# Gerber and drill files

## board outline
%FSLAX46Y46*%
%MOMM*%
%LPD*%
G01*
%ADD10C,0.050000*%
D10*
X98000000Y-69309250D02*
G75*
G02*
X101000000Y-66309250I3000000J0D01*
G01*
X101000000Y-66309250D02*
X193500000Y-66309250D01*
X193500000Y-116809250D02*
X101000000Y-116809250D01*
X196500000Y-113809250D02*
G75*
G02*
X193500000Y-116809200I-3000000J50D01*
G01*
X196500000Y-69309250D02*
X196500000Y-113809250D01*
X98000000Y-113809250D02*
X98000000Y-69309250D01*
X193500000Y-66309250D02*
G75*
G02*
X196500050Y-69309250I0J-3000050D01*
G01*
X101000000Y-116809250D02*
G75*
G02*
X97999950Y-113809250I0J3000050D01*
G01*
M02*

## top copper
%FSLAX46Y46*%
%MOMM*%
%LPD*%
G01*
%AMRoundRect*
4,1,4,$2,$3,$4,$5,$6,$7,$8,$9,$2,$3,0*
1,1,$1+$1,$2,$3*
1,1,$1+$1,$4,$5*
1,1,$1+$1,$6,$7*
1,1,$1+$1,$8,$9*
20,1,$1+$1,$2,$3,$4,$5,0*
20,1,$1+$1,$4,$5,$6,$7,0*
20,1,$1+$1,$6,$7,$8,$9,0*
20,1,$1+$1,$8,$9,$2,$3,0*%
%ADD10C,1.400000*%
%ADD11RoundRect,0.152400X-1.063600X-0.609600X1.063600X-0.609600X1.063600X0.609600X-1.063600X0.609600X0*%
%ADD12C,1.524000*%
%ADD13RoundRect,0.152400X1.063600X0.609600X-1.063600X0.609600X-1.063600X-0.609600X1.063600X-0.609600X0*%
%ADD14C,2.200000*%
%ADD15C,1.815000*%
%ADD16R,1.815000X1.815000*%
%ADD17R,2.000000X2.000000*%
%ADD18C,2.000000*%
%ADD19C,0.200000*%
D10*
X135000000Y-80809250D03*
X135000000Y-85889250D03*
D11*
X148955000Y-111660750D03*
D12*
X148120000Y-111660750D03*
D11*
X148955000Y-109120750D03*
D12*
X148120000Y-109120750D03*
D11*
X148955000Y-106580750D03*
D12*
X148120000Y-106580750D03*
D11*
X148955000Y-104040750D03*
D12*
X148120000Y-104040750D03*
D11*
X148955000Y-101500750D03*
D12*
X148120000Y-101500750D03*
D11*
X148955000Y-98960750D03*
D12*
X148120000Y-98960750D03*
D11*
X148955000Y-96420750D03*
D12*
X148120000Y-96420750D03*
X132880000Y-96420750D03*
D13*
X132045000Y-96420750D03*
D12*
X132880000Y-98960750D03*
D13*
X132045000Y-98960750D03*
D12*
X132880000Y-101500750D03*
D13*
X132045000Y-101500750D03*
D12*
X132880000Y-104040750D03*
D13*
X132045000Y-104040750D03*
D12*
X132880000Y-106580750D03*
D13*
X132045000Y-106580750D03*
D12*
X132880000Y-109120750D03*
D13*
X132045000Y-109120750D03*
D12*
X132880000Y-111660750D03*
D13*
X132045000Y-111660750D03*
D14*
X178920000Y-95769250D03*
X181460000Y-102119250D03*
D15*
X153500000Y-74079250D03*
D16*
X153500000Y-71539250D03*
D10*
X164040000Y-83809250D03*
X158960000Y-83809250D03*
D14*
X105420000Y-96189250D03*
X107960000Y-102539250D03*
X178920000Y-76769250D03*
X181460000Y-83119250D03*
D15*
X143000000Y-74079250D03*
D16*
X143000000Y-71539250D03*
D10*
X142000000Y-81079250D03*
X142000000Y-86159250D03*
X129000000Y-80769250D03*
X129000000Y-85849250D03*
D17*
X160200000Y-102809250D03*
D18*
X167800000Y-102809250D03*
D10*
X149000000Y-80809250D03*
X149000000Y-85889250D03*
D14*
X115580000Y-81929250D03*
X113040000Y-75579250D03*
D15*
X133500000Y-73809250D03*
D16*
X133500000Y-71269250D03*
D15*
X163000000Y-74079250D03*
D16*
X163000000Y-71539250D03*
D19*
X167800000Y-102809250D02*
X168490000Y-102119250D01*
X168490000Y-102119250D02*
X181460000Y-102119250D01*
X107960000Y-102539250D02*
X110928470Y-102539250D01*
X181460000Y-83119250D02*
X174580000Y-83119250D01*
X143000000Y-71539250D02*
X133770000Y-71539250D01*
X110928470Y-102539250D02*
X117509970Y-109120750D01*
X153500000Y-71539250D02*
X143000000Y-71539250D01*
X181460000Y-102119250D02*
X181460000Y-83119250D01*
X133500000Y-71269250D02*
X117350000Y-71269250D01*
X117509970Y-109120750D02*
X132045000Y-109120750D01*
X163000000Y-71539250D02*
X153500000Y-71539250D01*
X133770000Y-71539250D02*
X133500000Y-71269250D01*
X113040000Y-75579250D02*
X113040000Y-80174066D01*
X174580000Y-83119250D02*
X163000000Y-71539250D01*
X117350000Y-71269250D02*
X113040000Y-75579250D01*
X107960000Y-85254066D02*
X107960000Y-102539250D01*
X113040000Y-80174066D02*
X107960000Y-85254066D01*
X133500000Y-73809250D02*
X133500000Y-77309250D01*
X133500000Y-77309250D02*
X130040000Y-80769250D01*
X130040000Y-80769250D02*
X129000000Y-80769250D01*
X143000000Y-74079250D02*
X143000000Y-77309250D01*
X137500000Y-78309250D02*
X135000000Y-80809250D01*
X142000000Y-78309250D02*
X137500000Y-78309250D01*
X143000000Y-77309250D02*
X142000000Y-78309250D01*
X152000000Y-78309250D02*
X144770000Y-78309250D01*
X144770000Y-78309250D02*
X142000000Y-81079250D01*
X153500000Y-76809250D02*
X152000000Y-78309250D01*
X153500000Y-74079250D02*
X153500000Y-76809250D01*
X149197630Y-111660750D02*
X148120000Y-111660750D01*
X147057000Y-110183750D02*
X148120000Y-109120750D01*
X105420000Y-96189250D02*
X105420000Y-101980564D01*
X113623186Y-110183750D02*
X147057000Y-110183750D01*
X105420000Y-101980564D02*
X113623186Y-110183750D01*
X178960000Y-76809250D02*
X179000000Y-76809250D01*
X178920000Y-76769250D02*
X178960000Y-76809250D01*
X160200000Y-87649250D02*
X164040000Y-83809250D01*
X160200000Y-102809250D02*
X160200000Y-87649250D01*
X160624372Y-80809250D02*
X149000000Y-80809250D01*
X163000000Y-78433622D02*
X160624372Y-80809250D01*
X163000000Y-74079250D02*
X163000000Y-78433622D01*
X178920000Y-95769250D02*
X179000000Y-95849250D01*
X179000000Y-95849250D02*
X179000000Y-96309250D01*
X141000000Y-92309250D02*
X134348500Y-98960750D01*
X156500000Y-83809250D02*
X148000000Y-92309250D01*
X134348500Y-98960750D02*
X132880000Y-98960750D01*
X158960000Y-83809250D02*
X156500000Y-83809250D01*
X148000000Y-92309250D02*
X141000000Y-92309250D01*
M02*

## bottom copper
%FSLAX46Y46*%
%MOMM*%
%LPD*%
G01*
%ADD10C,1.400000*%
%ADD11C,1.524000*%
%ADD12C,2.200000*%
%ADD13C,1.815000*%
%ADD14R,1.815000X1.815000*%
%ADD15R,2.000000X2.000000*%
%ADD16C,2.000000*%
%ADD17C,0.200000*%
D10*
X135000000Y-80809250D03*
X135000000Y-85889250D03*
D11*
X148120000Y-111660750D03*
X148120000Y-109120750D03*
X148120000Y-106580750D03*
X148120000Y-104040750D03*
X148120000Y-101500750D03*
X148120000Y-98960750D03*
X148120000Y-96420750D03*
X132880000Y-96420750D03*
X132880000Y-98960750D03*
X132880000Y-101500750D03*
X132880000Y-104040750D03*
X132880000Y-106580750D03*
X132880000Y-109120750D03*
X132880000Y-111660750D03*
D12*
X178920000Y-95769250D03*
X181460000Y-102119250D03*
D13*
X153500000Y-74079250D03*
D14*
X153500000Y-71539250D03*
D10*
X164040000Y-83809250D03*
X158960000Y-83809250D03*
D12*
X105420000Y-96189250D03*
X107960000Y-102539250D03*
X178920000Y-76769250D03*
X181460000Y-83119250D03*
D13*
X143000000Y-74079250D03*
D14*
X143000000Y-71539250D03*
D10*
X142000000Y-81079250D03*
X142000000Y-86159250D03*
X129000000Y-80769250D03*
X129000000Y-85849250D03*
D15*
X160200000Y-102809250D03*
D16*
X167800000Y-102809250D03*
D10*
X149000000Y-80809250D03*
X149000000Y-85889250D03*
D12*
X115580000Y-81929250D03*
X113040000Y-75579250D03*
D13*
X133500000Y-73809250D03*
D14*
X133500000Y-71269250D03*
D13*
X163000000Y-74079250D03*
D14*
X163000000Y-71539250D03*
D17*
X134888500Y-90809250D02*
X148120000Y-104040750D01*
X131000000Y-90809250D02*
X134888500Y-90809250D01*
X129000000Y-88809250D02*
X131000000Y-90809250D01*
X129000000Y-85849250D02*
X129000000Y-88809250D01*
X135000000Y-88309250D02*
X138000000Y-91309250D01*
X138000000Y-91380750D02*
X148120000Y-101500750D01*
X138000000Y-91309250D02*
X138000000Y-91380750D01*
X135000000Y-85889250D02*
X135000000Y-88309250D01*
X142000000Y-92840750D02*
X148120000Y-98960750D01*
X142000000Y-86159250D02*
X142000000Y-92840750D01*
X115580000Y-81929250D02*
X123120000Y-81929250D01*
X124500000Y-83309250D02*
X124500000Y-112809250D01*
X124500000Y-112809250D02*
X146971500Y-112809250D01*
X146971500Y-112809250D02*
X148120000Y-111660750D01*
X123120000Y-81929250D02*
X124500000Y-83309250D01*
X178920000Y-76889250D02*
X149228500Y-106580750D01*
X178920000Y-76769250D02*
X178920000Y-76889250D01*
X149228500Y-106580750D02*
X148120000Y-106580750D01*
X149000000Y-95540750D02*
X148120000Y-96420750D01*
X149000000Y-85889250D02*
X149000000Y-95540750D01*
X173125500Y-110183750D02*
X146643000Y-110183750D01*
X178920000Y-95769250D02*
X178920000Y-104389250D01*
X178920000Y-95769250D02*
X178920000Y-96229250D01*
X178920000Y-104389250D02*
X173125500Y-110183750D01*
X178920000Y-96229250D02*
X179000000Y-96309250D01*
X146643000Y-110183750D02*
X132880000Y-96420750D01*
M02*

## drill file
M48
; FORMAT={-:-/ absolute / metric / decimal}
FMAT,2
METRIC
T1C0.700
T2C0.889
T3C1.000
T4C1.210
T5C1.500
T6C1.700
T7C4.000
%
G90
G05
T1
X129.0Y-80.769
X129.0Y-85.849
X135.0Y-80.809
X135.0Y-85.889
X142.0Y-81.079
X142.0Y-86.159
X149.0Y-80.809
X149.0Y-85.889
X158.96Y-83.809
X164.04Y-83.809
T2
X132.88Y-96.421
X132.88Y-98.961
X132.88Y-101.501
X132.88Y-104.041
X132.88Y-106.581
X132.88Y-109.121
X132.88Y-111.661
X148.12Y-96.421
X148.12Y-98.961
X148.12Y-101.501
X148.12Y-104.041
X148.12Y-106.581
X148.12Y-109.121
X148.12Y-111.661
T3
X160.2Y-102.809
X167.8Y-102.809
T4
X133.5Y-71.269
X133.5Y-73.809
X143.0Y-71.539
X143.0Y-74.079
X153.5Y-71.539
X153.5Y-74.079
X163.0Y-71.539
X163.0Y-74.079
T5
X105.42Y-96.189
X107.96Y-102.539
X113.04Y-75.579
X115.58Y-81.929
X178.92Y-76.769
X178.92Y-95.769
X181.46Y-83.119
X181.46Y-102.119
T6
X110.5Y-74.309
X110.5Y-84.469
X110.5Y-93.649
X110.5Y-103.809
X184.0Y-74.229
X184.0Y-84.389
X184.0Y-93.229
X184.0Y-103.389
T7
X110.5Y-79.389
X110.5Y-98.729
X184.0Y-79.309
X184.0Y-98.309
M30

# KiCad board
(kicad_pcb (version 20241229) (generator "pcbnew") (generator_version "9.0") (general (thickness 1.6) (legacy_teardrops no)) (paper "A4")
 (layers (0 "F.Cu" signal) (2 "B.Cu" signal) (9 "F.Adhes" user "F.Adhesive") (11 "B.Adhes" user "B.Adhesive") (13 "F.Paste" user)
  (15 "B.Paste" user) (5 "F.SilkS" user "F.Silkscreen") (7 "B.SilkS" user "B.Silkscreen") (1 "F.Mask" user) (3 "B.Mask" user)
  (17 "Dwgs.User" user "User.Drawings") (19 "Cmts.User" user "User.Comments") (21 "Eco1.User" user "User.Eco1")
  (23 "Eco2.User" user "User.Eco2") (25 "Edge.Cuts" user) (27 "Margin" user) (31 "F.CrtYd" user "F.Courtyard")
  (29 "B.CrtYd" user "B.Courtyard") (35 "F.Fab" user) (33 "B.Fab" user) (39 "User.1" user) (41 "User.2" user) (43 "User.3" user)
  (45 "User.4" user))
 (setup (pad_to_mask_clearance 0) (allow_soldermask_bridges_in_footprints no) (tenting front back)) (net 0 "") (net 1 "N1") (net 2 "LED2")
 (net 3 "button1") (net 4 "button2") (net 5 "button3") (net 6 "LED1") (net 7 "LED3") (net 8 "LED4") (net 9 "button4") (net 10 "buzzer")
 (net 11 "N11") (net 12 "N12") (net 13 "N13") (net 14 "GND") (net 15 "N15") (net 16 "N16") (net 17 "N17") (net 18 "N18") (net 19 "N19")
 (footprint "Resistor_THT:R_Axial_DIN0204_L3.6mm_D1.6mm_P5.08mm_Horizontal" (layer "F.Cu") (at 135 80.80925 -90)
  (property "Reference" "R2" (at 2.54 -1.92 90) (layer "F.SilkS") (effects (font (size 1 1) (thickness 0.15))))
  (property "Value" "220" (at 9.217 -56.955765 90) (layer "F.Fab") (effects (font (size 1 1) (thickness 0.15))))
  (pad "1" thru_hole circle (at 0 0 270) (size 1.4 1.4) (drill 0.7) (layers "*.Cu" "*.Mask") (remove_unused_layers no) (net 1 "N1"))
  (pad "2" thru_hole circle (at 5.08 0 270) (size 1.4 1.4) (drill 0.7) (layers "*.Cu" "*.Mask") (remove_unused_layers no) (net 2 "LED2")))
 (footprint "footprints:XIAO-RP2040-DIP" (layer "F.Cu") (at 140.5 104.04075 -90)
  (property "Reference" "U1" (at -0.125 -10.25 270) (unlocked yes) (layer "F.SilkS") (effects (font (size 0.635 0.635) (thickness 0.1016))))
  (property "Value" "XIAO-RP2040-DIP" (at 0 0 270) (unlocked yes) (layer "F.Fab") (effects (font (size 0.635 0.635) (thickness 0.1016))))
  (pad "1" smd roundrect (at 7.62 -8.455) (size 2.432 1.524) (layers "F.Cu" "F.Mask") (roundrect_rratio 0.1) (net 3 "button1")
   (thermal_bridge_angle 45))
  (pad "1" thru_hole circle (at 7.62 -7.62) (size 1.524 1.524) (drill 0.889) (layers "*.Cu" "*.Mask") (remove_unused_layers no)
   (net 3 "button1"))
  (pad "2" smd roundrect (at 5.08 -8.455) (size 2.432 1.524) (layers "F.Cu" "F.Mask") (roundrect_rratio 0.1) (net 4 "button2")
   (thermal_bridge_angle 45))
  (pad "2" thru_hole circle (at 5.08 -7.62) (size 1.524 1.524) (drill 0.889) (layers "*.Cu" "*.Mask") (remove_unused_layers no)
   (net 4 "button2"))
  (pad "3" smd roundrect (at 2.54 -8.455) (size 2.432 1.524) (layers "F.Cu" "F.Mask") (roundrect_rratio 0.1) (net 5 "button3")
   (thermal_bridge_angle 45))
  (pad "3" thru_hole circle (at 2.54 -7.62) (size 1.524 1.524) (drill 0.889) (layers "*.Cu" "*.Mask") (remove_unused_layers no)
   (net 5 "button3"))
  (pad "4" smd roundrect (at 0 -8.455) (size 2.432 1.524) (layers "F.Cu" "F.Mask") (roundrect_rratio 0.1) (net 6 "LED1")
   (thermal_bridge_angle 45))
  (pad "4" thru_hole circle (at 0 -7.62) (size 1.524 1.524) (drill 0.889) (layers "*.Cu" "*.Mask") (remove_unused_layers no) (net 6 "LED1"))
  (pad "5" smd roundrect (at -2.54 -8.455) (size 2.432 1.524) (layers "F.Cu" "F.Mask") (roundrect_rratio 0.1) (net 2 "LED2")
   (thermal_bridge_angle 45))
  (pad "5" thru_hole circle (at -2.54 -7.62) (size 1.524 1.524) (drill 0.889) (layers "*.Cu" "*.Mask") (remove_unused_layers no)
   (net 2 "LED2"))
  (pad "6" smd roundrect (at -5.08 -8.455) (size 2.432 1.524) (layers "F.Cu" "F.Mask") (roundrect_rratio 0.1) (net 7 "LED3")
   (thermal_bridge_angle 45))
  (pad "6" thru_hole circle (at -5.08 -7.62) (size 1.524 1.524) (drill 0.889) (layers "*.Cu" "*.Mask") (remove_unused_layers no)
   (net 7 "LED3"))
  (pad "7" smd roundrect (at -7.62 -8.455) (size 2.432 1.524) (layers "F.Cu" "F.Mask") (roundrect_rratio 0.1) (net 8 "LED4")
   (thermal_bridge_angle 45))
  (pad "7" thru_hole circle (at -7.62 -7.62) (size 1.524 1.524) (drill 0.889) (layers "*.Cu" "*.Mask") (remove_unused_layers no)
   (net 8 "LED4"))
  (pad "8" thru_hole circle (at -7.62 7.62 180) (size 1.524 1.524) (drill 0.889) (layers "*.Cu" "*.Mask") (remove_unused_layers no)
   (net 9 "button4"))
  (pad "8" smd roundrect (at -7.62 8.455 180) (size 2.432 1.524) (layers "F.Cu" "F.Mask") (roundrect_rratio 0.1) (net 9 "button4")
   (thermal_bridge_angle 45))
  (pad "9" thru_hole circle (at -5.08 7.62 180) (size 1.524 1.524) (drill 0.889) (layers "*.Cu" "*.Mask") (remove_unused_layers no)
   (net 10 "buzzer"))
  (pad "9" smd roundrect (at -5.08 8.455 180) (size 2.432 1.524) (layers "F.Cu" "F.Mask") (roundrect_rratio 0.1) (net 10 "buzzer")
   (thermal_bridge_angle 45))
  (pad "10" thru_hole circle (at -2.54 7.62 180) (size 1.524 1.524) (drill 0.889) (layers "*.Cu" "*.Mask") (remove_unused_layers no)
   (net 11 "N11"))
  (pad "10" smd roundrect (at -2.54 8.455 180) (size 2.432 1.524) (layers "F.Cu" "F.Mask") (roundrect_rratio 0.1) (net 11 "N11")
   (thermal_bridge_angle 45))
  (pad "11" thru_hole circle (at 0 7.62 180) (size 1.524 1.524) (drill 0.889) (layers "*.Cu" "*.Mask") (remove_unused_layers no)
   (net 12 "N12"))
  (pad "11" smd roundrect (at 0 8.455 180) (size 2.432 1.524) (layers "F.Cu" "F.Mask") (roundrect_rratio 0.1) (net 12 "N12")
   (thermal_bridge_angle 45))
  (pad "12" thru_hole circle (at 2.54 7.62 180) (size 1.524 1.524) (drill 0.889) (layers "*.Cu" "*.Mask") (remove_unused_layers no)
   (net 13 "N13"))
  (pad "12" smd roundrect (at 2.54 8.455 180) (size 2.432 1.524) (layers "F.Cu" "F.Mask") (roundrect_rratio 0.1) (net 13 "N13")
   (thermal_bridge_angle 45))
  (pad "13" thru_hole circle (at 5.08 7.62 180) (size 1.524 1.524) (drill 0.889) (layers "*.Cu" "*.Mask") (remove_unused_layers no)
   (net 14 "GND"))
  (pad "13" smd roundrect (at 5.08 8.455 180) (size 2.432 1.524) (layers "F.Cu" "F.Mask") (roundrect_rratio 0.1) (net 14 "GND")
   (thermal_bridge_angle 45))
  (pad "14" thru_hole circle (at 7.62 7.62 180) (size 1.524 1.524) (drill 0.889) (layers "*.Cu" "*.Mask") (remove_unused_layers no)
   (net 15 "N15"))
  (pad "14" smd roundrect (at 7.62 8.455 180) (size 2.432 1.524) (layers "F.Cu" "F.Mask") (roundrect_rratio 0.1) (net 15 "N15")
   (thermal_bridge_angle 45)))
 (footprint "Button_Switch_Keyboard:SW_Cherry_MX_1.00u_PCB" (layer "F.Cu") (at 178.92 95.76925 90)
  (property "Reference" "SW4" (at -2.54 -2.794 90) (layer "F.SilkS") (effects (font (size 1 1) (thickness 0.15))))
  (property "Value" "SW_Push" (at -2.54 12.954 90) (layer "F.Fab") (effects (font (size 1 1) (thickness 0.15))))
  (pad "" np_thru_hole circle (at -7.62 5.08 90) (size 1.7 1.7) (drill 1.7) (layers "*.Cu" "*.Mask"))
  (pad "" np_thru_hole circle (at -2.54 5.08 90) (size 4 4) (drill 4) (layers "*.Cu" "*.Mask"))
  (pad "" np_thru_hole circle (at 2.54 5.08 90) (size 1.7 1.7) (drill 1.7) (layers "*.Cu" "*.Mask"))
  (pad "1" thru_hole circle (at 0 0 90) (size 2.2 2.2) (drill 1.5) (layers "*.Cu" "*.Mask") (remove_unused_layers no) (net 9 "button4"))
  (pad "2" thru_hole circle (at -6.35 2.54 90) (size 2.2 2.2) (drill 1.5) (layers "*.Cu" "*.Mask") (remove_unused_layers no) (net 14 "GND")))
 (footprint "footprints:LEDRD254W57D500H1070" (layer "F.Cu") (at 153.5 72.80925 -90)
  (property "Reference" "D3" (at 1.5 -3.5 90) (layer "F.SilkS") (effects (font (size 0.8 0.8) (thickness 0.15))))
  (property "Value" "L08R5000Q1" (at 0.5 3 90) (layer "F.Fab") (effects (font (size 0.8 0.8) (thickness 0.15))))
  (pad "A" thru_hole circle (at 1.27 0 270) (size 1.815 1.815) (drill 1.21) (layers "*.Cu" "*.Mask") (remove_unused_layers no)
   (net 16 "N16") (solder_mask_margin 0.102))
  (pad "C" thru_hole rect (at -1.27 0 270) (size 1.815 1.815) (drill 1.21) (layers "*.Cu" "*.Mask") (remove_unused_layers no) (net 14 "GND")
   (solder_mask_margin 0.102)))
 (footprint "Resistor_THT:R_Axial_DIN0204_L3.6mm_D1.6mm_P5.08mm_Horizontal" (layer "F.Cu") (at 164.04 83.80925 180)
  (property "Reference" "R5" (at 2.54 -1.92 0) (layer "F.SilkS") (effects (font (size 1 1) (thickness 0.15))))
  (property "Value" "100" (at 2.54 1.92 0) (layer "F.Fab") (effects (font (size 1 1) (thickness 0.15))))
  (pad "1" thru_hole circle (at 0 0 180) (size 1.4 1.4) (drill 0.7) (layers "*.Cu" "*.Mask") (remove_unused_layers no) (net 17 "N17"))
  (pad "2" thru_hole circle (at 5.08 0 180) (size 1.4 1.4) (drill 0.7) (layers "*.Cu" "*.Mask") (remove_unused_layers no) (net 10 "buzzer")))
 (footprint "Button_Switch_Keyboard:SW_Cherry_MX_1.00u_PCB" (layer "F.Cu") (at 105.42 96.18925 90)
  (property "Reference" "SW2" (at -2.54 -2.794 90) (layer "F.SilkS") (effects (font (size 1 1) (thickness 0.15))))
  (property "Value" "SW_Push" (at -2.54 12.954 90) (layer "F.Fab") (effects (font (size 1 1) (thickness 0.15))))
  (pad "" np_thru_hole circle (at -7.62 5.08 90) (size 1.7 1.7) (drill 1.7) (layers "*.Cu" "*.Mask"))
  (pad "" np_thru_hole circle (at -2.54 5.08 90) (size 4 4) (drill 4) (layers "*.Cu" "*.Mask"))
  (pad "" np_thru_hole circle (at 2.54 5.08 90) (size 1.7 1.7) (drill 1.7) (layers "*.Cu" "*.Mask"))
  (pad "1" thru_hole circle (at 0 0 90) (size 2.2 2.2) (drill 1.5) (layers "*.Cu" "*.Mask") (remove_unused_layers no) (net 4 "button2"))
  (pad "2" thru_hole circle (at -6.35 2.54 90) (size 2.2 2.2) (drill 1.5) (layers "*.Cu" "*.Mask") (remove_unused_layers no) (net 14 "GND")))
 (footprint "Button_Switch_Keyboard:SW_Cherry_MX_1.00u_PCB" (layer "F.Cu") (at 178.92 76.76925 90)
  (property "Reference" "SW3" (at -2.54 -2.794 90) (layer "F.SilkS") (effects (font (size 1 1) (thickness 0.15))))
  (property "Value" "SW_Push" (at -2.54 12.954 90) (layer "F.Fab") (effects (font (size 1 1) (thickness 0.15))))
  (pad "" np_thru_hole circle (at -7.62 5.08 90) (size 1.7 1.7) (drill 1.7) (layers "*.Cu" "*.Mask"))
  (pad "" np_thru_hole circle (at -2.54 5.08 90) (size 4 4) (drill 4) (layers "*.Cu" "*.Mask"))
  (pad "" np_thru_hole circle (at 2.54 5.08 90) (size 1.7 1.7) (drill 1.7) (layers "*.Cu" "*.Mask"))
  (pad "1" thru_hole circle (at 0 0 90) (size 2.2 2.2) (drill 1.5) (layers "*.Cu" "*.Mask") (remove_unused_layers no) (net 5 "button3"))
  (pad "2" thru_hole circle (at -6.35 2.54 90) (size 2.2 2.2) (drill 1.5) (layers "*.Cu" "*.Mask") (remove_unused_layers no) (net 14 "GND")))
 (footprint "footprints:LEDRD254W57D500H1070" (layer "F.Cu") (at 143 72.80925 -90)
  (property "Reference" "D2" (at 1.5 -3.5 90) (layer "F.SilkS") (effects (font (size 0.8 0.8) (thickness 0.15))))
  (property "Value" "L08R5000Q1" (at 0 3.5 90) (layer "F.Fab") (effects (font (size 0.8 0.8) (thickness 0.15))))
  (pad "A" thru_hole circle (at 1.27 0 270) (size 1.815 1.815) (drill 1.21) (layers "*.Cu" "*.Mask") (remove_unused_layers no) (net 1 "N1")
   (solder_mask_margin 0.102))
  (pad "C" thru_hole rect (at -1.27 0 270) (size 1.815 1.815) (drill 1.21) (layers "*.Cu" "*.Mask") (remove_unused_layers no) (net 14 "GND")
   (solder_mask_margin 0.102)))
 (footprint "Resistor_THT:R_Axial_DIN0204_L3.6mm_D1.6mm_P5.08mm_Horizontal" (layer "F.Cu") (at 142 81.07925 -90)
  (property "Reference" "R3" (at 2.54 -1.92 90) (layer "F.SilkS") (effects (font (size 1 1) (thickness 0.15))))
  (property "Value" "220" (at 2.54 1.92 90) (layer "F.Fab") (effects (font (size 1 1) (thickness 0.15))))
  (pad "1" thru_hole circle (at 0 0 270) (size 1.4 1.4) (drill 0.7) (layers "*.Cu" "*.Mask") (remove_unused_layers no) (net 16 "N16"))
  (pad "2" thru_hole circle (at 5.08 0 270) (size 1.4 1.4) (drill 0.7) (layers "*.Cu" "*.Mask") (remove_unused_layers no) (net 7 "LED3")))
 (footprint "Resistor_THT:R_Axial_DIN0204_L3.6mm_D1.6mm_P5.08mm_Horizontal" (layer "F.Cu") (at 129 80.76925 -90)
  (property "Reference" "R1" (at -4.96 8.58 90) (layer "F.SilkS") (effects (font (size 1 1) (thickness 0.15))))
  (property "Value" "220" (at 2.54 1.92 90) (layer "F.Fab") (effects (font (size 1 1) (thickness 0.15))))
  (pad "1" thru_hole circle (at 0 0 270) (size 1.4 1.4) (drill 0.7) (layers "*.Cu" "*.Mask") (remove_unused_layers no) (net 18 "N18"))
  (pad "2" thru_hole circle (at 5.08 0 270) (size 1.4 1.4) (drill 0.7) (layers "*.Cu" "*.Mask") (remove_unused_layers no) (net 6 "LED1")))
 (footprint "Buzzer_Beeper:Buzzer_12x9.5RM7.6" (layer "F.Cu") (at 160.2 102.80925)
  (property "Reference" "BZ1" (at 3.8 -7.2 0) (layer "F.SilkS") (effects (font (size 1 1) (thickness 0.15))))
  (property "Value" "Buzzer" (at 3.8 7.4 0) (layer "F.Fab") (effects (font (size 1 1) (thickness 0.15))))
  (pad "1" thru_hole rect (at 0 0) (size 2 2) (drill 1) (layers "*.Cu" "*.Mask") (remove_unused_layers no) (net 17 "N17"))
  (pad "2" thru_hole circle (at 7.6 0) (size 2 2) (drill 1) (layers "*.Cu" "*.Mask") (remove_unused_layers no) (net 14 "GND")))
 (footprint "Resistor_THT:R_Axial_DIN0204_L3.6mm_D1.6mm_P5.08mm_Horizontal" (layer "F.Cu") (at 149 80.80925 -90)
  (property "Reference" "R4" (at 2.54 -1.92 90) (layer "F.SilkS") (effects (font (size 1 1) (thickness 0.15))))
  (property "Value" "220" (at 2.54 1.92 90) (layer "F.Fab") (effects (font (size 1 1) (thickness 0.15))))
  (pad "1" thru_hole circle (at 0 0 270) (size 1.4 1.4) (drill 0.7) (layers "*.Cu" "*.Mask") (remove_unused_layers no) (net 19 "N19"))
  (pad "2" thru_hole circle (at 5.08 0 270) (size 1.4 1.4) (drill 0.7) (layers "*.Cu" "*.Mask") (remove_unused_layers no) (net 8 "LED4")))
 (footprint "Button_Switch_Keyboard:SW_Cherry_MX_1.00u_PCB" (layer "F.Cu") (at 115.58 81.92925 -90)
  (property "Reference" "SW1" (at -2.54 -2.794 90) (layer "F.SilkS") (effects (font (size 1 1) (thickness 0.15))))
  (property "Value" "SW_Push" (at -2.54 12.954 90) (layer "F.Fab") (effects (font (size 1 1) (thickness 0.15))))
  (pad "" np_thru_hole circle (at -7.62 5.08 270) (size 1.7 1.7) (drill 1.7) (layers "*.Cu" "*.Mask"))
  (pad "" np_thru_hole circle (at -2.54 5.08 270) (size 4 4) (drill 4) (layers "*.Cu" "*.Mask"))
  (pad "" np_thru_hole circle (at 2.54 5.08 270) (size 1.7 1.7) (drill 1.7) (layers "*.Cu" "*.Mask"))
  (pad "1" thru_hole circle (at 0 0 270) (size 2.2 2.2) (drill 1.5) (layers "*.Cu" "*.Mask") (remove_unused_layers no) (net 3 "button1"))
  (pad "2" thru_hole circle (at -6.35 2.54 270) (size 2.2 2.2) (drill 1.5) (layers "*.Cu" "*.Mask") (remove_unused_layers no) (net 14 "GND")))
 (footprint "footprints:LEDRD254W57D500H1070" (layer "F.Cu") (at 133.5 72.53925 -90)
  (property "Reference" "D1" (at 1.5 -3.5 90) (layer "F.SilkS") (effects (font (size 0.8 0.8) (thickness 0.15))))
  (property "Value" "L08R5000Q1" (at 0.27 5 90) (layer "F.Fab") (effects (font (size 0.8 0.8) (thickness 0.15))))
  (pad "A" thru_hole circle (at 1.27 0 270) (size 1.815 1.815) (drill 1.21) (layers "*.Cu" "*.Mask") (remove_unused_layers no)
   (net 18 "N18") (solder_mask_margin 0.102))
  (pad "C" thru_hole rect (at -1.27 0 270) (size 1.815 1.815) (drill 1.21) (layers "*.Cu" "*.Mask") (remove_unused_layers no) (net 14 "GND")
   (solder_mask_margin 0.102)))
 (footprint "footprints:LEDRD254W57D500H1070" (layer "F.Cu") (at 163 72.80925 -90)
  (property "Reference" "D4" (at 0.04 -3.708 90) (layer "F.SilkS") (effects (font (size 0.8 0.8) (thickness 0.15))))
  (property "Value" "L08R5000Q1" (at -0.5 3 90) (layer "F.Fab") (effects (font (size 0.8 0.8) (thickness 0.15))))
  (pad "A" thru_hole circle (at 1.27 0 270) (size 1.815 1.815) (drill 1.21) (layers "*.Cu" "*.Mask") (remove_unused_layers no)
   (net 19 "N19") (solder_mask_margin 0.102))
  (pad "C" thru_hole rect (at -1.27 0 270) (size 1.815 1.815) (drill 1.21) (layers "*.Cu" "*.Mask") (remove_unused_layers no) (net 14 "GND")
   (solder_mask_margin 0.102)))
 (gr_arc (start 98 69.30925) (mid 98.87868 67.18793) (end 101 66.30925) (stroke (width 0.05) (type default)) (layer "Edge.Cuts"))
 (gr_line (start 101 66.30925) (end 193.5 66.30925) (stroke (width 0.05) (type default)) (layer "Edge.Cuts"))
 (gr_line (start 193.5 116.80925) (end 101 116.80925) (stroke (width 0.05) (type default)) (layer "Edge.Cuts"))
 (gr_arc (start 196.5 113.80925) (mid 195.62132 115.93057) (end 193.5 116.80925) (stroke (width 0.05) (type default)) (layer "Edge.Cuts"))
 (gr_line (start 196.5 69.30925) (end 196.5 113.80925) (stroke (width 0.05) (type default)) (layer "Edge.Cuts"))
 (gr_line (start 98 113.80925) (end 98 69.30925) (stroke (width 0.05) (type default)) (layer "Edge.Cuts"))
 (gr_arc (start 193.5 66.30925) (mid 195.62132 67.18793) (end 196.5 69.30925) (stroke (width 0.05) (type default)) (layer "Edge.Cuts"))
 (gr_arc (start 101 116.80925) (mid 98.87868 115.93057) (end 98 113.80925) (stroke (width 0.05) (type default)) (layer "Edge.Cuts"))
 (segment (start 167.8 102.80925) (end 168.49 102.11925) (width 0.2) (layer "F.Cu") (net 14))
 (segment (start 168.49 102.11925) (end 181.46 102.11925) (width 0.2) (layer "F.Cu") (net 14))
 (segment (start 107.96 102.53925) (end 110.92847 102.53925) (width 0.2) (layer "F.Cu") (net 14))
 (segment (start 181.46 83.11925) (end 174.58 83.11925) (width 0.2) (layer "F.Cu") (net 14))
 (segment (start 143 71.53925) (end 133.77 71.53925) (width 0.2) (layer "F.Cu") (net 14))
 (segment (start 110.92847 102.53925) (end 117.50997 109.12075) (width 0.2) (layer "F.Cu") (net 14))
 (segment (start 153.5 71.53925) (end 143 71.53925) (width 0.2) (layer "F.Cu") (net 14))
 (segment (start 181.46 102.11925) (end 181.46 83.11925) (width 0.2) (layer "F.Cu") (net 14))
 (segment (start 133.5 71.26925) (end 117.35 71.26925) (width 0.2) (layer "F.Cu") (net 14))
 (segment (start 117.50997 109.12075) (end 132.045 109.12075) (width 0.2) (layer "F.Cu") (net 14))
 (segment (start 163 71.53925) (end 153.5 71.53925) (width 0.2) (layer "F.Cu") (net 14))
 (segment (start 133.77 71.53925) (end 133.5 71.26925) (width 0.2) (layer "F.Cu") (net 14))
 (segment (start 113.04 75.57925) (end 113.04 80.174066) (width 0.2) (layer "F.Cu") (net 14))
 (segment (start 174.58 83.11925) (end 163 71.53925) (width 0.2) (layer "F.Cu") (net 14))
 (segment (start 117.35 71.26925) (end 113.04 75.57925) (width 0.2) (layer "F.Cu") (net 14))
 (segment (start 107.96 85.254066) (end 107.96 102.53925) (width 0.2) (layer "F.Cu") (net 14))
 (segment (start 113.04 80.174066) (end 107.96 85.254066) (width 0.2) (layer "F.Cu") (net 14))
 (segment (start 133.5 73.80925) (end 133.5 77.30925) (width 0.2) (layer "F.Cu") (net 18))
 (segment (start 133.5 77.30925) (end 130.04 80.76925) (width 0.2) (layer "F.Cu") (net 18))
 (segment (start 130.04 80.76925) (end 129 80.76925) (width 0.2) (layer "F.Cu") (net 18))
 (segment (start 143 74.07925) (end 143 77.30925) (width 0.2) (layer "F.Cu") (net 1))
 (segment (start 137.5 78.30925) (end 135 80.80925) (width 0.2) (layer "F.Cu") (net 1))
 (segment (start 142 78.30925) (end 137.5 78.30925) (width 0.2) (layer "F.Cu") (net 1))
 (segment (start 143 77.30925) (end 142 78.30925) (width 0.2) (layer "F.Cu") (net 1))
 (segment (start 152 78.30925) (end 144.77 78.30925) (width 0.2) (layer "F.Cu") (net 16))
 (segment (start 144.77 78.30925) (end 142 81.07925) (width 0.2) (layer "F.Cu") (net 16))
 (segment (start 153.5 76.80925) (end 152 78.30925) (width 0.2) (layer "F.Cu") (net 16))
 (segment (start 153.5 74.07925) (end 153.5 76.80925) (width 0.2) (layer "F.Cu") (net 16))
 (segment (start 134.8885 90.80925) (end 148.12 104.04075) (width 0.2) (layer "B.Cu") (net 6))
 (segment (start 131 90.80925) (end 134.8885 90.80925) (width 0.2) (layer "B.Cu") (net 6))
 (segment (start 129 88.80925) (end 131 90.80925) (width 0.2) (layer "B.Cu") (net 6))
 (segment (start 129 85.84925) (end 129 88.80925) (width 0.2) (layer "B.Cu") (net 6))
 (segment (start 135 88.30925) (end 138 91.30925) (width 0.2) (layer "B.Cu") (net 2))
 (segment (start 138 91.38075) (end 148.12 101.50075) (width 0.2) (layer "B.Cu") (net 2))
 (segment (start 138 91.30925) (end 138 91.38075) (width 0.2) (layer "B.Cu") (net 2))
 (segment (start 135 85.88925) (end 135 88.30925) (width 0.2) (layer "B.Cu") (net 2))
 (segment (start 142 92.84075) (end 148.12 98.96075) (width 0.2) (layer "B.Cu") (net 7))
 (segment (start 142 86.15925) (end 142 92.84075) (width 0.2) (layer "B.Cu") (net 7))
 (segment (start 149.19763 111.66075) (end 148.12 111.66075) (width 0.2) (layer "F.Cu") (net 3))
 (segment (start 115.58 81.92925) (end 123.12 81.92925) (width 0.2) (layer "B.Cu") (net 3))
 (segment (start 124.5 83.30925) (end 124.5 112.80925) (width 0.2) (layer "B.Cu") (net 3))
 (segment (start 124.5 112.80925) (end 146.9715 112.80925) (width 0.2) (layer "B.Cu") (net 3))
 (segment (start 146.9715 112.80925) (end 148.12 111.66075) (width 0.2) (layer "B.Cu") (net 3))
 (segment (start 123.12 81.92925) (end 124.5 83.30925) (width 0.2) (layer "B.Cu") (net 3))
 (segment (start 147.057 110.18375) (end 148.12 109.12075) (width 0.2) (layer "F.Cu") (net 4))
 (segment (start 105.42 96.18925) (end 105.42 101.980564) (width 0.2) (layer "F.Cu") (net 4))
 (segment (start 113.623186 110.18375) (end 147.057 110.18375) (width 0.2) (layer "F.Cu") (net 4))
 (segment (start 105.42 101.980564) (end 113.623186 110.18375) (width 0.2) (layer "F.Cu") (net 4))
 (segment (start 178.96 76.80925) (end 179 76.80925) (width 0.2) (layer "F.Cu") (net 5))
 (segment (start 178.92 76.76925) (end 178.96 76.80925) (width 0.2) (layer "F.Cu") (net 5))
 (segment (start 178.92 76.88925) (end 149.2285 106.58075) (width 0.2) (layer "B.Cu") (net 5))
 (segment (start 178.92 76.76925) (end 178.92 76.88925) (width 0.2) (layer "B.Cu") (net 5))
 (segment (start 149.2285 106.58075) (end 148.12 106.58075) (width 0.2) (layer "B.Cu") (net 5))
 (segment (start 160.2 87.64925) (end 164.04 83.80925) (width 0.2) (layer "F.Cu") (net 17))
 (segment (start 160.2 102.80925) (end 160.2 87.64925) (width 0.2) (layer "F.Cu") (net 17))
 (segment (start 160.624372 80.80925) (end 149 80.80925) (width 0.2) (layer "F.Cu") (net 19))
 (segment (start 163 78.433622) (end 160.624372 80.80925) (width 0.2) (layer "F.Cu") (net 19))
 (segment (start 163 74.07925) (end 163 78.433622) (width 0.2) (layer "F.Cu") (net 19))
 (segment (start 149 95.54075) (end 148.12 96.42075) (width 0.2) (layer "B.Cu") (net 8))
 (segment (start 149 85.88925) (end 149 95.54075) (width 0.2) (layer "B.Cu") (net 8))
 (segment (start 178.92 95.76925) (end 179 95.84925) (width 0.2) (layer "F.Cu") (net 9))
 (segment (start 179 95.84925) (end 179 96.30925) (width 0.2) (layer "F.Cu") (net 9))
 (segment (start 173.1255 110.18375) (end 146.643 110.18375) (width 0.2) (layer "B.Cu") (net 9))
 (segment (start 178.92 95.76925) (end 178.92 104.38925) (width 0.2) (layer "B.Cu") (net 9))
 (segment (start 178.92 95.76925) (end 178.92 96.22925) (width 0.2) (layer "B.Cu") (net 9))
 (segment (start 178.92 104.38925) (end 173.1255 110.18375) (width 0.2) (layer "B.Cu") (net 9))
 (segment (start 178.92 96.22925) (end 179 96.30925) (width 0.2) (layer "B.Cu") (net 9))
 (segment (start 146.643 110.18375) (end 132.88 96.42075) (width 0.2) (layer "B.Cu") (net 9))
 (segment (start 141 92.30925) (end 134.3485 98.96075) (width 0.2) (layer "F.Cu") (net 10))
 (segment (start 156.5 83.80925) (end 148 92.30925) (width 0.2) (layer "F.Cu") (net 10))
 (segment (start 134.3485 98.96075) (end 132.88 98.96075) (width 0.2) (layer "F.Cu") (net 10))
 (segment (start 158.96 83.80925) (end 156.5 83.80925) (width 0.2) (layer "F.Cu") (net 10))
 (segment (start 148 92.30925) (end 141 92.30925) (width 0.2) (layer "F.Cu") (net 10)))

